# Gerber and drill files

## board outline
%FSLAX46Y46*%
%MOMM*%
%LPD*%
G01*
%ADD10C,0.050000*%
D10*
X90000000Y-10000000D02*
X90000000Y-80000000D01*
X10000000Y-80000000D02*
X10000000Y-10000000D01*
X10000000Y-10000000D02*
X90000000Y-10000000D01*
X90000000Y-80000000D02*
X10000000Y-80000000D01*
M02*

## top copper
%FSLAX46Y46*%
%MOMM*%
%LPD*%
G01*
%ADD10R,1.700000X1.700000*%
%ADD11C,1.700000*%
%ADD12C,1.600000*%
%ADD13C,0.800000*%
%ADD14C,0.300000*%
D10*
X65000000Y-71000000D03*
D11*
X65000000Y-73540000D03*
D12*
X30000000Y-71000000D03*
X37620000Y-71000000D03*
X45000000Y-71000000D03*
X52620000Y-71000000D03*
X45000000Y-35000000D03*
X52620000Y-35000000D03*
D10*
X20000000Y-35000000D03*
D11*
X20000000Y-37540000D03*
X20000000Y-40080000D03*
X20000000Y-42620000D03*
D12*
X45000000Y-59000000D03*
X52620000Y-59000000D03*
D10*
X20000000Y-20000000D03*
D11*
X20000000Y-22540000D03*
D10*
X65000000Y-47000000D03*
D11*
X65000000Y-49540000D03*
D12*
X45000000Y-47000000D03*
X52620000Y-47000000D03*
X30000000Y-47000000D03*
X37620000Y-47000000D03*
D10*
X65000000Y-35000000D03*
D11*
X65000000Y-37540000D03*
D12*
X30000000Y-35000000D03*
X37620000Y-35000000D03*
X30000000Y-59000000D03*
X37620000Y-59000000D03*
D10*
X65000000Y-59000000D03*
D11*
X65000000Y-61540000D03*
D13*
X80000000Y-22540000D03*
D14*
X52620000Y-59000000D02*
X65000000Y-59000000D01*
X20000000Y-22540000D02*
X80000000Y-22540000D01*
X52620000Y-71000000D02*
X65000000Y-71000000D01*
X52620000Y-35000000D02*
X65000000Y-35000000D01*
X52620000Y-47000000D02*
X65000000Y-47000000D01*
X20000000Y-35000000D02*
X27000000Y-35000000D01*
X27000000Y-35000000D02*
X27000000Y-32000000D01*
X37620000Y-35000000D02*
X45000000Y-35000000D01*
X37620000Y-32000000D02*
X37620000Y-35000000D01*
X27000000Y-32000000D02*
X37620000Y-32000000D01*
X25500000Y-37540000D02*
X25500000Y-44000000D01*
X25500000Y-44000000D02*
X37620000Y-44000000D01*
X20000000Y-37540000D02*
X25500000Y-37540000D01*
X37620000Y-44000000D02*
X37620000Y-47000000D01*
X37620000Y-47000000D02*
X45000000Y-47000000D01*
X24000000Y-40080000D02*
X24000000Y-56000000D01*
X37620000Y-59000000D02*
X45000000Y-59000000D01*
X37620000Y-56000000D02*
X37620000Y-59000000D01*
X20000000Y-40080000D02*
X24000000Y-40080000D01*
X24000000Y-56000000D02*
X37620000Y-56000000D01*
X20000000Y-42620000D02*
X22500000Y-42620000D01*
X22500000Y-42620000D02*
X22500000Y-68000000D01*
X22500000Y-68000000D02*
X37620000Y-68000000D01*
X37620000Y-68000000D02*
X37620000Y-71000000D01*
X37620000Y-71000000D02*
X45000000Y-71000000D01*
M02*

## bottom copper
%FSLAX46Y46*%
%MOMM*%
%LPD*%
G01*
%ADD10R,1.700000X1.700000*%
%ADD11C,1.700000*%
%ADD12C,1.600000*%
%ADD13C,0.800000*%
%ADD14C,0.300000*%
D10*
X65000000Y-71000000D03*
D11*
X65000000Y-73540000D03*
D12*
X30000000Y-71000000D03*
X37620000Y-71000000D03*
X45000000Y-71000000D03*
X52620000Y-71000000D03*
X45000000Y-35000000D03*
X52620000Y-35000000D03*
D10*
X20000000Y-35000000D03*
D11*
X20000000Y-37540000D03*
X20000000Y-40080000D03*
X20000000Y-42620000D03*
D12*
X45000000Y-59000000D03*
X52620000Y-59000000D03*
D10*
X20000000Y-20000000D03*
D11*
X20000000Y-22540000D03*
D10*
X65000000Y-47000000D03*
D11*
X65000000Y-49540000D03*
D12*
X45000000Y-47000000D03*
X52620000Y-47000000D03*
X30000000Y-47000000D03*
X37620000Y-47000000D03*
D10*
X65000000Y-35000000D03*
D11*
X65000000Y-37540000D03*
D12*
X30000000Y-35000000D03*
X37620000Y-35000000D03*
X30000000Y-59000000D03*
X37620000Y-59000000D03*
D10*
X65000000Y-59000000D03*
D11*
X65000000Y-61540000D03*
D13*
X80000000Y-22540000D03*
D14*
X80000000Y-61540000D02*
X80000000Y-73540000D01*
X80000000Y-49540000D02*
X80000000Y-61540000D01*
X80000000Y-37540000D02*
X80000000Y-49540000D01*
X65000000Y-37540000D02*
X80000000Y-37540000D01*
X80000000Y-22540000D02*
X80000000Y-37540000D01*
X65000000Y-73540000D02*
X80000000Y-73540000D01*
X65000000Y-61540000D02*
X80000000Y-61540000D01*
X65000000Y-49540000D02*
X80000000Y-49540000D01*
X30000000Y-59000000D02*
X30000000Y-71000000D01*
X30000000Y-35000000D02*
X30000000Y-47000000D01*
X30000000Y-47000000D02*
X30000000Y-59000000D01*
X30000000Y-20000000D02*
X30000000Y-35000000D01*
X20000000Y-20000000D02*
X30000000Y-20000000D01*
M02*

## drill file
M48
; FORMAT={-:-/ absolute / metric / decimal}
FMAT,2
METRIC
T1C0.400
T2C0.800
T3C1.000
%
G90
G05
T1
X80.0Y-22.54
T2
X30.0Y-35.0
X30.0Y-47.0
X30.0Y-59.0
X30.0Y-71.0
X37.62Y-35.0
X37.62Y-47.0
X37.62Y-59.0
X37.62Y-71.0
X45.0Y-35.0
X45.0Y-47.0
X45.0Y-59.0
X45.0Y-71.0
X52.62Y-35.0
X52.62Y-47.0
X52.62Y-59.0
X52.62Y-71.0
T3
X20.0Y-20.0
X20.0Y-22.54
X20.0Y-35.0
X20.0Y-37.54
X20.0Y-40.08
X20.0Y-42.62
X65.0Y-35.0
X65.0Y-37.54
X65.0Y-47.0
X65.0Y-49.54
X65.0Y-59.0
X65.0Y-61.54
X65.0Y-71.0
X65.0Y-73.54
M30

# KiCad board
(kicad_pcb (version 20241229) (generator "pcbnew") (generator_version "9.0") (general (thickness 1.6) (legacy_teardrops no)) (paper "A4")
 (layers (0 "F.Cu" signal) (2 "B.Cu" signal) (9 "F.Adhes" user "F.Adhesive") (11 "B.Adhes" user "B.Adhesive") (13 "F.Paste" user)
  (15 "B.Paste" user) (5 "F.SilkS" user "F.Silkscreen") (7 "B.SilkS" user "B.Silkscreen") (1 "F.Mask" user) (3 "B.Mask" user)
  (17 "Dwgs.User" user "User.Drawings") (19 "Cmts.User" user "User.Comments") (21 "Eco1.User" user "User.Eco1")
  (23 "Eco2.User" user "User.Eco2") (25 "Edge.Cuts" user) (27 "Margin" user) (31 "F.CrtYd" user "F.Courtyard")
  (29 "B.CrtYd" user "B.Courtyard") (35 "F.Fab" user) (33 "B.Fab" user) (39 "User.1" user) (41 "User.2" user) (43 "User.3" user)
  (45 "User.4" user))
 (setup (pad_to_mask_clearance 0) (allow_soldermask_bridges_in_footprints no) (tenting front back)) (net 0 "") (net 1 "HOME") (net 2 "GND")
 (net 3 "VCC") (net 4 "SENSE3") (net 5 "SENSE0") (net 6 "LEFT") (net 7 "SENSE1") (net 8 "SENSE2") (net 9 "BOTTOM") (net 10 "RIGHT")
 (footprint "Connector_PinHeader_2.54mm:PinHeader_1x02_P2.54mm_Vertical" (layer "F.Cu") (at 65 71)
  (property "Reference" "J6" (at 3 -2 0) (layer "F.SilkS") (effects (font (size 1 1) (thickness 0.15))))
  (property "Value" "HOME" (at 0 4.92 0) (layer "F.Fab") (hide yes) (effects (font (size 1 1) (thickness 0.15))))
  (pad "1" thru_hole rect (at 0 0) (size 1.7 1.7) (drill 1) (layers "*.Cu" "*.Mask") (remove_unused_layers no) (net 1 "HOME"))
  (pad "2" thru_hole circle (at 0 2.54) (size 1.7 1.7) (drill 1) (layers "*.Cu" "*.Mask") (remove_unused_layers no) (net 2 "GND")))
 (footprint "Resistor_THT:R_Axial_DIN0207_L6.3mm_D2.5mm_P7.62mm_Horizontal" (layer "F.Cu") (at 30 71)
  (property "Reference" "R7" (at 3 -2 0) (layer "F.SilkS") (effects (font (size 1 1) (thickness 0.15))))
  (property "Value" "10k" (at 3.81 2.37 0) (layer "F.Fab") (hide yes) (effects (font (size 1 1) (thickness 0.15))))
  (pad "1" thru_hole circle (at 0 0) (size 1.6 1.6) (drill 0.8) (layers "*.Cu" "*.Mask") (remove_unused_layers no) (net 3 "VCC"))
  (pad "2" thru_hole circle (at 7.62 0) (size 1.6 1.6) (drill 0.8) (layers "*.Cu" "*.Mask") (remove_unused_layers no) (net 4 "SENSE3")))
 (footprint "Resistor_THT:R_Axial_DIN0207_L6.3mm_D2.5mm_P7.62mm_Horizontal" (layer "F.Cu") (at 45 71)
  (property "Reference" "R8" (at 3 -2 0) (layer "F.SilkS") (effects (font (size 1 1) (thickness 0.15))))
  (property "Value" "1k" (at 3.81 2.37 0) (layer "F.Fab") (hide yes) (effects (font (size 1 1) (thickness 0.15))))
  (pad "1" thru_hole circle (at 0 0) (size 1.6 1.6) (drill 0.8) (layers "*.Cu" "*.Mask") (remove_unused_layers no) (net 4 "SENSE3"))
  (pad "2" thru_hole circle (at 7.62 0) (size 1.6 1.6) (drill 0.8) (layers "*.Cu" "*.Mask") (remove_unused_layers no) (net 1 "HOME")))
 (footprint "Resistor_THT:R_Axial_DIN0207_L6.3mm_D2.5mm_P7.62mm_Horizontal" (layer "F.Cu") (at 45 35)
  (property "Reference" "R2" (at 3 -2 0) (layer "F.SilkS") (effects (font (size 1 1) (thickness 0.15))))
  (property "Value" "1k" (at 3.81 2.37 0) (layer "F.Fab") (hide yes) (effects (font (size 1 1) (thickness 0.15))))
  (pad "1" thru_hole circle (at 0 0) (size 1.6 1.6) (drill 0.8) (layers "*.Cu" "*.Mask") (remove_unused_layers no) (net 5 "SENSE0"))
  (pad "2" thru_hole circle (at 7.62 0) (size 1.6 1.6) (drill 0.8) (layers "*.Cu" "*.Mask") (remove_unused_layers no) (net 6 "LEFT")))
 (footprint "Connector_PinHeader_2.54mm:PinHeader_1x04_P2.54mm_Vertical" (layer "F.Cu") (at 20 35)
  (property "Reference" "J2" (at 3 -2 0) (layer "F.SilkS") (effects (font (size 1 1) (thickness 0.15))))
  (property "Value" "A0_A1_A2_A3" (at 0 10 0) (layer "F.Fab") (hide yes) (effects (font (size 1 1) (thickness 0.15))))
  (pad "1" thru_hole rect (at 0 0) (size 1.7 1.7) (drill 1) (layers "*.Cu" "*.Mask") (remove_unused_layers no) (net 5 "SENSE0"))
  (pad "2" thru_hole circle (at 0 2.54) (size 1.7 1.7) (drill 1) (layers "*.Cu" "*.Mask") (remove_unused_layers no) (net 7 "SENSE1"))
  (pad "3" thru_hole circle (at 0 5.08) (size 1.7 1.7) (drill 1) (layers "*.Cu" "*.Mask") (remove_unused_layers no) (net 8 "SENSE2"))
  (pad "4" thru_hole circle (at 0 7.62) (size 1.7 1.7) (drill 1) (layers "*.Cu" "*.Mask") (remove_unused_layers no) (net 4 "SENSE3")))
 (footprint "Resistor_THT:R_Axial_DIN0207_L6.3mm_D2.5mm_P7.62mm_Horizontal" (layer "F.Cu") (at 45 59)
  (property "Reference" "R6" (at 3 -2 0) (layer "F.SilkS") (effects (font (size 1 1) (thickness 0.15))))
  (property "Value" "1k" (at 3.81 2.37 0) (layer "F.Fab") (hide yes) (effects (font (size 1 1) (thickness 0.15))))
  (pad "1" thru_hole circle (at 0 0) (size 1.6 1.6) (drill 0.8) (layers "*.Cu" "*.Mask") (remove_unused_layers no) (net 8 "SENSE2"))
  (pad "2" thru_hole circle (at 7.62 0) (size 1.6 1.6) (drill 0.8) (layers "*.Cu" "*.Mask") (remove_unused_layers no) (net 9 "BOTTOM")))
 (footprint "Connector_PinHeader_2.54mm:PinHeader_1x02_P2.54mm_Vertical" (layer "F.Cu") (at 20 20)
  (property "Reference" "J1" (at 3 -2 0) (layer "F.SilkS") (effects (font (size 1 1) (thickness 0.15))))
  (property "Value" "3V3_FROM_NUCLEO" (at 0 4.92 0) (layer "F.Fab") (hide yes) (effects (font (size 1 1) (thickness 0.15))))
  (pad "1" thru_hole rect (at 0 0) (size 1.7 1.7) (drill 1) (layers "*.Cu" "*.Mask") (remove_unused_layers no) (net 3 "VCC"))
  (pad "2" thru_hole circle (at 0 2.54) (size 1.7 1.7) (drill 1) (layers "*.Cu" "*.Mask") (remove_unused_layers no) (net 2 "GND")))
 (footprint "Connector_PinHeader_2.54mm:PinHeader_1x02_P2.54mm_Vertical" (layer "F.Cu") (at 65 47)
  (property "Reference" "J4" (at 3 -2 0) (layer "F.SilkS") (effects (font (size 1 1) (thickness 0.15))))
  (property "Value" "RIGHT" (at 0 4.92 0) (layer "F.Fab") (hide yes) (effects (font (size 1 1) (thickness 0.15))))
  (pad "1" thru_hole rect (at 0 0) (size 1.7 1.7) (drill 1) (layers "*.Cu" "*.Mask") (remove_unused_layers no) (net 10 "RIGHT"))
  (pad "2" thru_hole circle (at 0 2.54) (size 1.7 1.7) (drill 1) (layers "*.Cu" "*.Mask") (remove_unused_layers no) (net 2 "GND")))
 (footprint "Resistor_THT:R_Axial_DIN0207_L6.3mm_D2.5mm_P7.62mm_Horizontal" (layer "F.Cu") (at 45 47)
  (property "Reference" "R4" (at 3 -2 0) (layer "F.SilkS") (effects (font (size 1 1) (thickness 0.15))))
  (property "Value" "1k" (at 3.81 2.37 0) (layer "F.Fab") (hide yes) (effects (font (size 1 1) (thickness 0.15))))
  (pad "1" thru_hole circle (at 0 0) (size 1.6 1.6) (drill 0.8) (layers "*.Cu" "*.Mask") (remove_unused_layers no) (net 7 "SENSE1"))
  (pad "2" thru_hole circle (at 7.62 0) (size 1.6 1.6) (drill 0.8) (layers "*.Cu" "*.Mask") (remove_unused_layers no) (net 10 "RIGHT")))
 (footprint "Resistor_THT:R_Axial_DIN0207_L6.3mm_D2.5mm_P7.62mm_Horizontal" (layer "F.Cu") (at 30 47)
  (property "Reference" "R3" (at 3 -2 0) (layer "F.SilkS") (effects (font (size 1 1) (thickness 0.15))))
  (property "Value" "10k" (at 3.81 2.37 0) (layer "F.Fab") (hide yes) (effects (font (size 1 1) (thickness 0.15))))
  (pad "1" thru_hole circle (at 0 0) (size 1.6 1.6) (drill 0.8) (layers "*.Cu" "*.Mask") (remove_unused_layers no) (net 3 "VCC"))
  (pad "2" thru_hole circle (at 7.62 0) (size 1.6 1.6) (drill 0.8) (layers "*.Cu" "*.Mask") (remove_unused_layers no) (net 7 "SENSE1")))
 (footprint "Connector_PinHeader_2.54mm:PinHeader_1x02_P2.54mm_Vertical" (layer "F.Cu") (at 65 35)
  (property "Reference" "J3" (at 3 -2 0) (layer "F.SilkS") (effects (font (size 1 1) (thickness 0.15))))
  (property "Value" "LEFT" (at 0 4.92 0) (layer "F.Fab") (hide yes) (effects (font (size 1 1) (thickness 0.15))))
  (pad "1" thru_hole rect (at 0 0) (size 1.7 1.7) (drill 1) (layers "*.Cu" "*.Mask") (remove_unused_layers no) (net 6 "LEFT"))
  (pad "2" thru_hole circle (at 0 2.54) (size 1.7 1.7) (drill 1) (layers "*.Cu" "*.Mask") (remove_unused_layers no) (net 2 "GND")))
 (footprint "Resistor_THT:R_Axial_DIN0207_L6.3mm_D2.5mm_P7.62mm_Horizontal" (layer "F.Cu") (at 30 35)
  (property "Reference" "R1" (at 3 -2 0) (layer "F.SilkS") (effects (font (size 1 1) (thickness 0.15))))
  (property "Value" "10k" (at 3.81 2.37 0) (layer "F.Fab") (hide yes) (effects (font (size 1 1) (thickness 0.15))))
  (pad "1" thru_hole circle (at 0 0) (size 1.6 1.6) (drill 0.8) (layers "*.Cu" "*.Mask") (remove_unused_layers no) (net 3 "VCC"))
  (pad "2" thru_hole circle (at 7.62 0) (size 1.6 1.6) (drill 0.8) (layers "*.Cu" "*.Mask") (remove_unused_layers no) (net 5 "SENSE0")))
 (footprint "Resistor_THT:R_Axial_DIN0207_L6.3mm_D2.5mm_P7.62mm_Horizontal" (layer "F.Cu") (at 30 59)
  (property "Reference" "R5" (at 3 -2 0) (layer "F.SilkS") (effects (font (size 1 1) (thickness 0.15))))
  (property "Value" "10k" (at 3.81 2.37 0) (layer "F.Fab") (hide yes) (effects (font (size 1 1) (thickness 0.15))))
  (pad "1" thru_hole circle (at 0 0) (size 1.6 1.6) (drill 0.8) (layers "*.Cu" "*.Mask") (remove_unused_layers no) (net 3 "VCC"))
  (pad "2" thru_hole circle (at 7.62 0) (size 1.6 1.6) (drill 0.8) (layers "*.Cu" "*.Mask") (remove_unused_layers no) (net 8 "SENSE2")))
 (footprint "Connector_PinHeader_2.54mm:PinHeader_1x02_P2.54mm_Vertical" (layer "F.Cu") (at 65 59)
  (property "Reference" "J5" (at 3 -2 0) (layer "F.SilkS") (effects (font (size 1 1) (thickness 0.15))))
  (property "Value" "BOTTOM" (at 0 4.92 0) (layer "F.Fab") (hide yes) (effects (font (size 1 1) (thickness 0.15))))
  (pad "1" thru_hole rect (at 0 0) (size 1.7 1.7) (drill 1) (layers "*.Cu" "*.Mask") (remove_unused_layers no) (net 9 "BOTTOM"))
  (pad "2" thru_hole circle (at 0 2.54) (size 1.7 1.7) (drill 1) (layers "*.Cu" "*.Mask") (remove_unused_layers no) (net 2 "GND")))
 (gr_line (start 90 10) (end 90 80) (stroke (width 0.05) (type default)) (layer "Edge.Cuts"))
 (gr_line (start 10 80) (end 10 10) (stroke (width 0.05) (type default)) (layer "Edge.Cuts"))
 (gr_line (start 10 10) (end 90 10) (stroke (width 0.05) (type default)) (layer "Edge.Cuts"))
 (gr_line (start 90 80) (end 10 80) (stroke (width 0.05) (type default)) (layer "Edge.Cuts"))
 (segment (start 52.62 59) (end 65 59) (width 0.3) (layer "F.Cu") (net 9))
 (segment (start 20 22.54) (end 80 22.54) (width 0.3) (layer "F.Cu") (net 2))
 (via (at 80 22.54) (size 0.8) (drill 0.4) (layers "F.Cu" "B.Cu") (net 2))
 (segment (start 80 61.54) (end 80 73.54) (width 0.3) (layer "B.Cu") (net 2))
 (segment (start 80 49.54) (end 80 61.54) (width 0.3) (layer "B.Cu") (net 2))
 (segment (start 80 37.54) (end 80 49.54) (width 0.3) (layer "B.Cu") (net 2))
 (segment (start 65 37.54) (end 80 37.54) (width 0.3) (layer "B.Cu") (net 2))
 (segment (start 80 22.54) (end 80 37.54) (width 0.3) (layer "B.Cu") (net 2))
 (segment (start 65 73.54) (end 80 73.54) (width 0.3) (layer "B.Cu") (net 2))
 (segment (start 65 61.54) (end 80 61.54) (width 0.3) (layer "B.Cu") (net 2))
 (segment (start 65 49.54) (end 80 49.54) (width 0.3) (layer "B.Cu") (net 2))
 (segment (start 52.62 71) (end 65 71) (width 0.3) (layer "F.Cu") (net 1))
 (segment (start 52.62 35) (end 65 35) (width 0.3) (layer "F.Cu") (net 6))
 (segment (start 52.62 47) (end 65 47) (width 0.3) (layer "F.Cu") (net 10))
 (segment (start 20 35) (end 27 35) (width 0.3) (layer "F.Cu") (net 5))
 (segment (start 27 35) (end 27 32) (width 0.3) (layer "F.Cu") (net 5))
 (segment (start 37.62 35) (end 45 35) (width 0.3) (layer "F.Cu") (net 5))
 (segment (start 37.62 32) (end 37.62 35) (width 0.3) (layer "F.Cu") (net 5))
 (segment (start 27 32) (end 37.62 32) (width 0.3) (layer "F.Cu") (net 5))
 (segment (start 25.5 37.54) (end 25.5 44) (width 0.3) (layer "F.Cu") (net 7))
 (segment (start 25.5 44) (end 37.62 44) (width 0.3) (layer "F.Cu") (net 7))
 (segment (start 20 37.54) (end 25.5 37.54) (width 0.3) (layer "F.Cu") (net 7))
 (segment (start 37.62 44) (end 37.62 47) (width 0.3) (layer "F.Cu") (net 7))
 (segment (start 37.62 47) (end 45 47) (width 0.3) (layer "F.Cu") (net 7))
 (segment (start 24 40.08) (end 24 56) (width 0.3) (layer "F.Cu") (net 8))
 (segment (start 37.62 59) (end 45 59) (width 0.3) (layer "F.Cu") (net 8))
 (segment (start 37.62 56) (end 37.62 59) (width 0.3) (layer "F.Cu") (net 8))
 (segment (start 20 40.08) (end 24 40.08) (width 0.3) (layer "F.Cu") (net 8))
 (segment (start 24 56) (end 37.62 56) (width 0.3) (layer "F.Cu") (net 8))
 (segment (start 20 42.62) (end 22.5 42.62) (width 0.3) (layer "F.Cu") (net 4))
 (segment (start 22.5 42.62) (end 22.5 68) (width 0.3) (layer "F.Cu") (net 4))
 (segment (start 22.5 68) (end 37.62 68) (width 0.3) (layer "F.Cu") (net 4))
 (segment (start 37.62 68) (end 37.62 71) (width 0.3) (layer "F.Cu") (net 4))
 (segment (start 37.62 71) (end 45 71) (width 0.3) (layer "F.Cu") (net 4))
 (segment (start 30 59) (end 30 71) (width 0.3) (layer "B.Cu") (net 3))
 (segment (start 30 35) (end 30 47) (width 0.3) (layer "B.Cu") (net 3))
 (segment (start 30 47) (end 30 59) (width 0.3) (layer "B.Cu") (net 3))
 (segment (start 30 20) (end 30 35) (width 0.3) (layer "B.Cu") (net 3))
 (segment (start 20 20) (end 30 20) (width 0.3) (layer "B.Cu") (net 3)))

